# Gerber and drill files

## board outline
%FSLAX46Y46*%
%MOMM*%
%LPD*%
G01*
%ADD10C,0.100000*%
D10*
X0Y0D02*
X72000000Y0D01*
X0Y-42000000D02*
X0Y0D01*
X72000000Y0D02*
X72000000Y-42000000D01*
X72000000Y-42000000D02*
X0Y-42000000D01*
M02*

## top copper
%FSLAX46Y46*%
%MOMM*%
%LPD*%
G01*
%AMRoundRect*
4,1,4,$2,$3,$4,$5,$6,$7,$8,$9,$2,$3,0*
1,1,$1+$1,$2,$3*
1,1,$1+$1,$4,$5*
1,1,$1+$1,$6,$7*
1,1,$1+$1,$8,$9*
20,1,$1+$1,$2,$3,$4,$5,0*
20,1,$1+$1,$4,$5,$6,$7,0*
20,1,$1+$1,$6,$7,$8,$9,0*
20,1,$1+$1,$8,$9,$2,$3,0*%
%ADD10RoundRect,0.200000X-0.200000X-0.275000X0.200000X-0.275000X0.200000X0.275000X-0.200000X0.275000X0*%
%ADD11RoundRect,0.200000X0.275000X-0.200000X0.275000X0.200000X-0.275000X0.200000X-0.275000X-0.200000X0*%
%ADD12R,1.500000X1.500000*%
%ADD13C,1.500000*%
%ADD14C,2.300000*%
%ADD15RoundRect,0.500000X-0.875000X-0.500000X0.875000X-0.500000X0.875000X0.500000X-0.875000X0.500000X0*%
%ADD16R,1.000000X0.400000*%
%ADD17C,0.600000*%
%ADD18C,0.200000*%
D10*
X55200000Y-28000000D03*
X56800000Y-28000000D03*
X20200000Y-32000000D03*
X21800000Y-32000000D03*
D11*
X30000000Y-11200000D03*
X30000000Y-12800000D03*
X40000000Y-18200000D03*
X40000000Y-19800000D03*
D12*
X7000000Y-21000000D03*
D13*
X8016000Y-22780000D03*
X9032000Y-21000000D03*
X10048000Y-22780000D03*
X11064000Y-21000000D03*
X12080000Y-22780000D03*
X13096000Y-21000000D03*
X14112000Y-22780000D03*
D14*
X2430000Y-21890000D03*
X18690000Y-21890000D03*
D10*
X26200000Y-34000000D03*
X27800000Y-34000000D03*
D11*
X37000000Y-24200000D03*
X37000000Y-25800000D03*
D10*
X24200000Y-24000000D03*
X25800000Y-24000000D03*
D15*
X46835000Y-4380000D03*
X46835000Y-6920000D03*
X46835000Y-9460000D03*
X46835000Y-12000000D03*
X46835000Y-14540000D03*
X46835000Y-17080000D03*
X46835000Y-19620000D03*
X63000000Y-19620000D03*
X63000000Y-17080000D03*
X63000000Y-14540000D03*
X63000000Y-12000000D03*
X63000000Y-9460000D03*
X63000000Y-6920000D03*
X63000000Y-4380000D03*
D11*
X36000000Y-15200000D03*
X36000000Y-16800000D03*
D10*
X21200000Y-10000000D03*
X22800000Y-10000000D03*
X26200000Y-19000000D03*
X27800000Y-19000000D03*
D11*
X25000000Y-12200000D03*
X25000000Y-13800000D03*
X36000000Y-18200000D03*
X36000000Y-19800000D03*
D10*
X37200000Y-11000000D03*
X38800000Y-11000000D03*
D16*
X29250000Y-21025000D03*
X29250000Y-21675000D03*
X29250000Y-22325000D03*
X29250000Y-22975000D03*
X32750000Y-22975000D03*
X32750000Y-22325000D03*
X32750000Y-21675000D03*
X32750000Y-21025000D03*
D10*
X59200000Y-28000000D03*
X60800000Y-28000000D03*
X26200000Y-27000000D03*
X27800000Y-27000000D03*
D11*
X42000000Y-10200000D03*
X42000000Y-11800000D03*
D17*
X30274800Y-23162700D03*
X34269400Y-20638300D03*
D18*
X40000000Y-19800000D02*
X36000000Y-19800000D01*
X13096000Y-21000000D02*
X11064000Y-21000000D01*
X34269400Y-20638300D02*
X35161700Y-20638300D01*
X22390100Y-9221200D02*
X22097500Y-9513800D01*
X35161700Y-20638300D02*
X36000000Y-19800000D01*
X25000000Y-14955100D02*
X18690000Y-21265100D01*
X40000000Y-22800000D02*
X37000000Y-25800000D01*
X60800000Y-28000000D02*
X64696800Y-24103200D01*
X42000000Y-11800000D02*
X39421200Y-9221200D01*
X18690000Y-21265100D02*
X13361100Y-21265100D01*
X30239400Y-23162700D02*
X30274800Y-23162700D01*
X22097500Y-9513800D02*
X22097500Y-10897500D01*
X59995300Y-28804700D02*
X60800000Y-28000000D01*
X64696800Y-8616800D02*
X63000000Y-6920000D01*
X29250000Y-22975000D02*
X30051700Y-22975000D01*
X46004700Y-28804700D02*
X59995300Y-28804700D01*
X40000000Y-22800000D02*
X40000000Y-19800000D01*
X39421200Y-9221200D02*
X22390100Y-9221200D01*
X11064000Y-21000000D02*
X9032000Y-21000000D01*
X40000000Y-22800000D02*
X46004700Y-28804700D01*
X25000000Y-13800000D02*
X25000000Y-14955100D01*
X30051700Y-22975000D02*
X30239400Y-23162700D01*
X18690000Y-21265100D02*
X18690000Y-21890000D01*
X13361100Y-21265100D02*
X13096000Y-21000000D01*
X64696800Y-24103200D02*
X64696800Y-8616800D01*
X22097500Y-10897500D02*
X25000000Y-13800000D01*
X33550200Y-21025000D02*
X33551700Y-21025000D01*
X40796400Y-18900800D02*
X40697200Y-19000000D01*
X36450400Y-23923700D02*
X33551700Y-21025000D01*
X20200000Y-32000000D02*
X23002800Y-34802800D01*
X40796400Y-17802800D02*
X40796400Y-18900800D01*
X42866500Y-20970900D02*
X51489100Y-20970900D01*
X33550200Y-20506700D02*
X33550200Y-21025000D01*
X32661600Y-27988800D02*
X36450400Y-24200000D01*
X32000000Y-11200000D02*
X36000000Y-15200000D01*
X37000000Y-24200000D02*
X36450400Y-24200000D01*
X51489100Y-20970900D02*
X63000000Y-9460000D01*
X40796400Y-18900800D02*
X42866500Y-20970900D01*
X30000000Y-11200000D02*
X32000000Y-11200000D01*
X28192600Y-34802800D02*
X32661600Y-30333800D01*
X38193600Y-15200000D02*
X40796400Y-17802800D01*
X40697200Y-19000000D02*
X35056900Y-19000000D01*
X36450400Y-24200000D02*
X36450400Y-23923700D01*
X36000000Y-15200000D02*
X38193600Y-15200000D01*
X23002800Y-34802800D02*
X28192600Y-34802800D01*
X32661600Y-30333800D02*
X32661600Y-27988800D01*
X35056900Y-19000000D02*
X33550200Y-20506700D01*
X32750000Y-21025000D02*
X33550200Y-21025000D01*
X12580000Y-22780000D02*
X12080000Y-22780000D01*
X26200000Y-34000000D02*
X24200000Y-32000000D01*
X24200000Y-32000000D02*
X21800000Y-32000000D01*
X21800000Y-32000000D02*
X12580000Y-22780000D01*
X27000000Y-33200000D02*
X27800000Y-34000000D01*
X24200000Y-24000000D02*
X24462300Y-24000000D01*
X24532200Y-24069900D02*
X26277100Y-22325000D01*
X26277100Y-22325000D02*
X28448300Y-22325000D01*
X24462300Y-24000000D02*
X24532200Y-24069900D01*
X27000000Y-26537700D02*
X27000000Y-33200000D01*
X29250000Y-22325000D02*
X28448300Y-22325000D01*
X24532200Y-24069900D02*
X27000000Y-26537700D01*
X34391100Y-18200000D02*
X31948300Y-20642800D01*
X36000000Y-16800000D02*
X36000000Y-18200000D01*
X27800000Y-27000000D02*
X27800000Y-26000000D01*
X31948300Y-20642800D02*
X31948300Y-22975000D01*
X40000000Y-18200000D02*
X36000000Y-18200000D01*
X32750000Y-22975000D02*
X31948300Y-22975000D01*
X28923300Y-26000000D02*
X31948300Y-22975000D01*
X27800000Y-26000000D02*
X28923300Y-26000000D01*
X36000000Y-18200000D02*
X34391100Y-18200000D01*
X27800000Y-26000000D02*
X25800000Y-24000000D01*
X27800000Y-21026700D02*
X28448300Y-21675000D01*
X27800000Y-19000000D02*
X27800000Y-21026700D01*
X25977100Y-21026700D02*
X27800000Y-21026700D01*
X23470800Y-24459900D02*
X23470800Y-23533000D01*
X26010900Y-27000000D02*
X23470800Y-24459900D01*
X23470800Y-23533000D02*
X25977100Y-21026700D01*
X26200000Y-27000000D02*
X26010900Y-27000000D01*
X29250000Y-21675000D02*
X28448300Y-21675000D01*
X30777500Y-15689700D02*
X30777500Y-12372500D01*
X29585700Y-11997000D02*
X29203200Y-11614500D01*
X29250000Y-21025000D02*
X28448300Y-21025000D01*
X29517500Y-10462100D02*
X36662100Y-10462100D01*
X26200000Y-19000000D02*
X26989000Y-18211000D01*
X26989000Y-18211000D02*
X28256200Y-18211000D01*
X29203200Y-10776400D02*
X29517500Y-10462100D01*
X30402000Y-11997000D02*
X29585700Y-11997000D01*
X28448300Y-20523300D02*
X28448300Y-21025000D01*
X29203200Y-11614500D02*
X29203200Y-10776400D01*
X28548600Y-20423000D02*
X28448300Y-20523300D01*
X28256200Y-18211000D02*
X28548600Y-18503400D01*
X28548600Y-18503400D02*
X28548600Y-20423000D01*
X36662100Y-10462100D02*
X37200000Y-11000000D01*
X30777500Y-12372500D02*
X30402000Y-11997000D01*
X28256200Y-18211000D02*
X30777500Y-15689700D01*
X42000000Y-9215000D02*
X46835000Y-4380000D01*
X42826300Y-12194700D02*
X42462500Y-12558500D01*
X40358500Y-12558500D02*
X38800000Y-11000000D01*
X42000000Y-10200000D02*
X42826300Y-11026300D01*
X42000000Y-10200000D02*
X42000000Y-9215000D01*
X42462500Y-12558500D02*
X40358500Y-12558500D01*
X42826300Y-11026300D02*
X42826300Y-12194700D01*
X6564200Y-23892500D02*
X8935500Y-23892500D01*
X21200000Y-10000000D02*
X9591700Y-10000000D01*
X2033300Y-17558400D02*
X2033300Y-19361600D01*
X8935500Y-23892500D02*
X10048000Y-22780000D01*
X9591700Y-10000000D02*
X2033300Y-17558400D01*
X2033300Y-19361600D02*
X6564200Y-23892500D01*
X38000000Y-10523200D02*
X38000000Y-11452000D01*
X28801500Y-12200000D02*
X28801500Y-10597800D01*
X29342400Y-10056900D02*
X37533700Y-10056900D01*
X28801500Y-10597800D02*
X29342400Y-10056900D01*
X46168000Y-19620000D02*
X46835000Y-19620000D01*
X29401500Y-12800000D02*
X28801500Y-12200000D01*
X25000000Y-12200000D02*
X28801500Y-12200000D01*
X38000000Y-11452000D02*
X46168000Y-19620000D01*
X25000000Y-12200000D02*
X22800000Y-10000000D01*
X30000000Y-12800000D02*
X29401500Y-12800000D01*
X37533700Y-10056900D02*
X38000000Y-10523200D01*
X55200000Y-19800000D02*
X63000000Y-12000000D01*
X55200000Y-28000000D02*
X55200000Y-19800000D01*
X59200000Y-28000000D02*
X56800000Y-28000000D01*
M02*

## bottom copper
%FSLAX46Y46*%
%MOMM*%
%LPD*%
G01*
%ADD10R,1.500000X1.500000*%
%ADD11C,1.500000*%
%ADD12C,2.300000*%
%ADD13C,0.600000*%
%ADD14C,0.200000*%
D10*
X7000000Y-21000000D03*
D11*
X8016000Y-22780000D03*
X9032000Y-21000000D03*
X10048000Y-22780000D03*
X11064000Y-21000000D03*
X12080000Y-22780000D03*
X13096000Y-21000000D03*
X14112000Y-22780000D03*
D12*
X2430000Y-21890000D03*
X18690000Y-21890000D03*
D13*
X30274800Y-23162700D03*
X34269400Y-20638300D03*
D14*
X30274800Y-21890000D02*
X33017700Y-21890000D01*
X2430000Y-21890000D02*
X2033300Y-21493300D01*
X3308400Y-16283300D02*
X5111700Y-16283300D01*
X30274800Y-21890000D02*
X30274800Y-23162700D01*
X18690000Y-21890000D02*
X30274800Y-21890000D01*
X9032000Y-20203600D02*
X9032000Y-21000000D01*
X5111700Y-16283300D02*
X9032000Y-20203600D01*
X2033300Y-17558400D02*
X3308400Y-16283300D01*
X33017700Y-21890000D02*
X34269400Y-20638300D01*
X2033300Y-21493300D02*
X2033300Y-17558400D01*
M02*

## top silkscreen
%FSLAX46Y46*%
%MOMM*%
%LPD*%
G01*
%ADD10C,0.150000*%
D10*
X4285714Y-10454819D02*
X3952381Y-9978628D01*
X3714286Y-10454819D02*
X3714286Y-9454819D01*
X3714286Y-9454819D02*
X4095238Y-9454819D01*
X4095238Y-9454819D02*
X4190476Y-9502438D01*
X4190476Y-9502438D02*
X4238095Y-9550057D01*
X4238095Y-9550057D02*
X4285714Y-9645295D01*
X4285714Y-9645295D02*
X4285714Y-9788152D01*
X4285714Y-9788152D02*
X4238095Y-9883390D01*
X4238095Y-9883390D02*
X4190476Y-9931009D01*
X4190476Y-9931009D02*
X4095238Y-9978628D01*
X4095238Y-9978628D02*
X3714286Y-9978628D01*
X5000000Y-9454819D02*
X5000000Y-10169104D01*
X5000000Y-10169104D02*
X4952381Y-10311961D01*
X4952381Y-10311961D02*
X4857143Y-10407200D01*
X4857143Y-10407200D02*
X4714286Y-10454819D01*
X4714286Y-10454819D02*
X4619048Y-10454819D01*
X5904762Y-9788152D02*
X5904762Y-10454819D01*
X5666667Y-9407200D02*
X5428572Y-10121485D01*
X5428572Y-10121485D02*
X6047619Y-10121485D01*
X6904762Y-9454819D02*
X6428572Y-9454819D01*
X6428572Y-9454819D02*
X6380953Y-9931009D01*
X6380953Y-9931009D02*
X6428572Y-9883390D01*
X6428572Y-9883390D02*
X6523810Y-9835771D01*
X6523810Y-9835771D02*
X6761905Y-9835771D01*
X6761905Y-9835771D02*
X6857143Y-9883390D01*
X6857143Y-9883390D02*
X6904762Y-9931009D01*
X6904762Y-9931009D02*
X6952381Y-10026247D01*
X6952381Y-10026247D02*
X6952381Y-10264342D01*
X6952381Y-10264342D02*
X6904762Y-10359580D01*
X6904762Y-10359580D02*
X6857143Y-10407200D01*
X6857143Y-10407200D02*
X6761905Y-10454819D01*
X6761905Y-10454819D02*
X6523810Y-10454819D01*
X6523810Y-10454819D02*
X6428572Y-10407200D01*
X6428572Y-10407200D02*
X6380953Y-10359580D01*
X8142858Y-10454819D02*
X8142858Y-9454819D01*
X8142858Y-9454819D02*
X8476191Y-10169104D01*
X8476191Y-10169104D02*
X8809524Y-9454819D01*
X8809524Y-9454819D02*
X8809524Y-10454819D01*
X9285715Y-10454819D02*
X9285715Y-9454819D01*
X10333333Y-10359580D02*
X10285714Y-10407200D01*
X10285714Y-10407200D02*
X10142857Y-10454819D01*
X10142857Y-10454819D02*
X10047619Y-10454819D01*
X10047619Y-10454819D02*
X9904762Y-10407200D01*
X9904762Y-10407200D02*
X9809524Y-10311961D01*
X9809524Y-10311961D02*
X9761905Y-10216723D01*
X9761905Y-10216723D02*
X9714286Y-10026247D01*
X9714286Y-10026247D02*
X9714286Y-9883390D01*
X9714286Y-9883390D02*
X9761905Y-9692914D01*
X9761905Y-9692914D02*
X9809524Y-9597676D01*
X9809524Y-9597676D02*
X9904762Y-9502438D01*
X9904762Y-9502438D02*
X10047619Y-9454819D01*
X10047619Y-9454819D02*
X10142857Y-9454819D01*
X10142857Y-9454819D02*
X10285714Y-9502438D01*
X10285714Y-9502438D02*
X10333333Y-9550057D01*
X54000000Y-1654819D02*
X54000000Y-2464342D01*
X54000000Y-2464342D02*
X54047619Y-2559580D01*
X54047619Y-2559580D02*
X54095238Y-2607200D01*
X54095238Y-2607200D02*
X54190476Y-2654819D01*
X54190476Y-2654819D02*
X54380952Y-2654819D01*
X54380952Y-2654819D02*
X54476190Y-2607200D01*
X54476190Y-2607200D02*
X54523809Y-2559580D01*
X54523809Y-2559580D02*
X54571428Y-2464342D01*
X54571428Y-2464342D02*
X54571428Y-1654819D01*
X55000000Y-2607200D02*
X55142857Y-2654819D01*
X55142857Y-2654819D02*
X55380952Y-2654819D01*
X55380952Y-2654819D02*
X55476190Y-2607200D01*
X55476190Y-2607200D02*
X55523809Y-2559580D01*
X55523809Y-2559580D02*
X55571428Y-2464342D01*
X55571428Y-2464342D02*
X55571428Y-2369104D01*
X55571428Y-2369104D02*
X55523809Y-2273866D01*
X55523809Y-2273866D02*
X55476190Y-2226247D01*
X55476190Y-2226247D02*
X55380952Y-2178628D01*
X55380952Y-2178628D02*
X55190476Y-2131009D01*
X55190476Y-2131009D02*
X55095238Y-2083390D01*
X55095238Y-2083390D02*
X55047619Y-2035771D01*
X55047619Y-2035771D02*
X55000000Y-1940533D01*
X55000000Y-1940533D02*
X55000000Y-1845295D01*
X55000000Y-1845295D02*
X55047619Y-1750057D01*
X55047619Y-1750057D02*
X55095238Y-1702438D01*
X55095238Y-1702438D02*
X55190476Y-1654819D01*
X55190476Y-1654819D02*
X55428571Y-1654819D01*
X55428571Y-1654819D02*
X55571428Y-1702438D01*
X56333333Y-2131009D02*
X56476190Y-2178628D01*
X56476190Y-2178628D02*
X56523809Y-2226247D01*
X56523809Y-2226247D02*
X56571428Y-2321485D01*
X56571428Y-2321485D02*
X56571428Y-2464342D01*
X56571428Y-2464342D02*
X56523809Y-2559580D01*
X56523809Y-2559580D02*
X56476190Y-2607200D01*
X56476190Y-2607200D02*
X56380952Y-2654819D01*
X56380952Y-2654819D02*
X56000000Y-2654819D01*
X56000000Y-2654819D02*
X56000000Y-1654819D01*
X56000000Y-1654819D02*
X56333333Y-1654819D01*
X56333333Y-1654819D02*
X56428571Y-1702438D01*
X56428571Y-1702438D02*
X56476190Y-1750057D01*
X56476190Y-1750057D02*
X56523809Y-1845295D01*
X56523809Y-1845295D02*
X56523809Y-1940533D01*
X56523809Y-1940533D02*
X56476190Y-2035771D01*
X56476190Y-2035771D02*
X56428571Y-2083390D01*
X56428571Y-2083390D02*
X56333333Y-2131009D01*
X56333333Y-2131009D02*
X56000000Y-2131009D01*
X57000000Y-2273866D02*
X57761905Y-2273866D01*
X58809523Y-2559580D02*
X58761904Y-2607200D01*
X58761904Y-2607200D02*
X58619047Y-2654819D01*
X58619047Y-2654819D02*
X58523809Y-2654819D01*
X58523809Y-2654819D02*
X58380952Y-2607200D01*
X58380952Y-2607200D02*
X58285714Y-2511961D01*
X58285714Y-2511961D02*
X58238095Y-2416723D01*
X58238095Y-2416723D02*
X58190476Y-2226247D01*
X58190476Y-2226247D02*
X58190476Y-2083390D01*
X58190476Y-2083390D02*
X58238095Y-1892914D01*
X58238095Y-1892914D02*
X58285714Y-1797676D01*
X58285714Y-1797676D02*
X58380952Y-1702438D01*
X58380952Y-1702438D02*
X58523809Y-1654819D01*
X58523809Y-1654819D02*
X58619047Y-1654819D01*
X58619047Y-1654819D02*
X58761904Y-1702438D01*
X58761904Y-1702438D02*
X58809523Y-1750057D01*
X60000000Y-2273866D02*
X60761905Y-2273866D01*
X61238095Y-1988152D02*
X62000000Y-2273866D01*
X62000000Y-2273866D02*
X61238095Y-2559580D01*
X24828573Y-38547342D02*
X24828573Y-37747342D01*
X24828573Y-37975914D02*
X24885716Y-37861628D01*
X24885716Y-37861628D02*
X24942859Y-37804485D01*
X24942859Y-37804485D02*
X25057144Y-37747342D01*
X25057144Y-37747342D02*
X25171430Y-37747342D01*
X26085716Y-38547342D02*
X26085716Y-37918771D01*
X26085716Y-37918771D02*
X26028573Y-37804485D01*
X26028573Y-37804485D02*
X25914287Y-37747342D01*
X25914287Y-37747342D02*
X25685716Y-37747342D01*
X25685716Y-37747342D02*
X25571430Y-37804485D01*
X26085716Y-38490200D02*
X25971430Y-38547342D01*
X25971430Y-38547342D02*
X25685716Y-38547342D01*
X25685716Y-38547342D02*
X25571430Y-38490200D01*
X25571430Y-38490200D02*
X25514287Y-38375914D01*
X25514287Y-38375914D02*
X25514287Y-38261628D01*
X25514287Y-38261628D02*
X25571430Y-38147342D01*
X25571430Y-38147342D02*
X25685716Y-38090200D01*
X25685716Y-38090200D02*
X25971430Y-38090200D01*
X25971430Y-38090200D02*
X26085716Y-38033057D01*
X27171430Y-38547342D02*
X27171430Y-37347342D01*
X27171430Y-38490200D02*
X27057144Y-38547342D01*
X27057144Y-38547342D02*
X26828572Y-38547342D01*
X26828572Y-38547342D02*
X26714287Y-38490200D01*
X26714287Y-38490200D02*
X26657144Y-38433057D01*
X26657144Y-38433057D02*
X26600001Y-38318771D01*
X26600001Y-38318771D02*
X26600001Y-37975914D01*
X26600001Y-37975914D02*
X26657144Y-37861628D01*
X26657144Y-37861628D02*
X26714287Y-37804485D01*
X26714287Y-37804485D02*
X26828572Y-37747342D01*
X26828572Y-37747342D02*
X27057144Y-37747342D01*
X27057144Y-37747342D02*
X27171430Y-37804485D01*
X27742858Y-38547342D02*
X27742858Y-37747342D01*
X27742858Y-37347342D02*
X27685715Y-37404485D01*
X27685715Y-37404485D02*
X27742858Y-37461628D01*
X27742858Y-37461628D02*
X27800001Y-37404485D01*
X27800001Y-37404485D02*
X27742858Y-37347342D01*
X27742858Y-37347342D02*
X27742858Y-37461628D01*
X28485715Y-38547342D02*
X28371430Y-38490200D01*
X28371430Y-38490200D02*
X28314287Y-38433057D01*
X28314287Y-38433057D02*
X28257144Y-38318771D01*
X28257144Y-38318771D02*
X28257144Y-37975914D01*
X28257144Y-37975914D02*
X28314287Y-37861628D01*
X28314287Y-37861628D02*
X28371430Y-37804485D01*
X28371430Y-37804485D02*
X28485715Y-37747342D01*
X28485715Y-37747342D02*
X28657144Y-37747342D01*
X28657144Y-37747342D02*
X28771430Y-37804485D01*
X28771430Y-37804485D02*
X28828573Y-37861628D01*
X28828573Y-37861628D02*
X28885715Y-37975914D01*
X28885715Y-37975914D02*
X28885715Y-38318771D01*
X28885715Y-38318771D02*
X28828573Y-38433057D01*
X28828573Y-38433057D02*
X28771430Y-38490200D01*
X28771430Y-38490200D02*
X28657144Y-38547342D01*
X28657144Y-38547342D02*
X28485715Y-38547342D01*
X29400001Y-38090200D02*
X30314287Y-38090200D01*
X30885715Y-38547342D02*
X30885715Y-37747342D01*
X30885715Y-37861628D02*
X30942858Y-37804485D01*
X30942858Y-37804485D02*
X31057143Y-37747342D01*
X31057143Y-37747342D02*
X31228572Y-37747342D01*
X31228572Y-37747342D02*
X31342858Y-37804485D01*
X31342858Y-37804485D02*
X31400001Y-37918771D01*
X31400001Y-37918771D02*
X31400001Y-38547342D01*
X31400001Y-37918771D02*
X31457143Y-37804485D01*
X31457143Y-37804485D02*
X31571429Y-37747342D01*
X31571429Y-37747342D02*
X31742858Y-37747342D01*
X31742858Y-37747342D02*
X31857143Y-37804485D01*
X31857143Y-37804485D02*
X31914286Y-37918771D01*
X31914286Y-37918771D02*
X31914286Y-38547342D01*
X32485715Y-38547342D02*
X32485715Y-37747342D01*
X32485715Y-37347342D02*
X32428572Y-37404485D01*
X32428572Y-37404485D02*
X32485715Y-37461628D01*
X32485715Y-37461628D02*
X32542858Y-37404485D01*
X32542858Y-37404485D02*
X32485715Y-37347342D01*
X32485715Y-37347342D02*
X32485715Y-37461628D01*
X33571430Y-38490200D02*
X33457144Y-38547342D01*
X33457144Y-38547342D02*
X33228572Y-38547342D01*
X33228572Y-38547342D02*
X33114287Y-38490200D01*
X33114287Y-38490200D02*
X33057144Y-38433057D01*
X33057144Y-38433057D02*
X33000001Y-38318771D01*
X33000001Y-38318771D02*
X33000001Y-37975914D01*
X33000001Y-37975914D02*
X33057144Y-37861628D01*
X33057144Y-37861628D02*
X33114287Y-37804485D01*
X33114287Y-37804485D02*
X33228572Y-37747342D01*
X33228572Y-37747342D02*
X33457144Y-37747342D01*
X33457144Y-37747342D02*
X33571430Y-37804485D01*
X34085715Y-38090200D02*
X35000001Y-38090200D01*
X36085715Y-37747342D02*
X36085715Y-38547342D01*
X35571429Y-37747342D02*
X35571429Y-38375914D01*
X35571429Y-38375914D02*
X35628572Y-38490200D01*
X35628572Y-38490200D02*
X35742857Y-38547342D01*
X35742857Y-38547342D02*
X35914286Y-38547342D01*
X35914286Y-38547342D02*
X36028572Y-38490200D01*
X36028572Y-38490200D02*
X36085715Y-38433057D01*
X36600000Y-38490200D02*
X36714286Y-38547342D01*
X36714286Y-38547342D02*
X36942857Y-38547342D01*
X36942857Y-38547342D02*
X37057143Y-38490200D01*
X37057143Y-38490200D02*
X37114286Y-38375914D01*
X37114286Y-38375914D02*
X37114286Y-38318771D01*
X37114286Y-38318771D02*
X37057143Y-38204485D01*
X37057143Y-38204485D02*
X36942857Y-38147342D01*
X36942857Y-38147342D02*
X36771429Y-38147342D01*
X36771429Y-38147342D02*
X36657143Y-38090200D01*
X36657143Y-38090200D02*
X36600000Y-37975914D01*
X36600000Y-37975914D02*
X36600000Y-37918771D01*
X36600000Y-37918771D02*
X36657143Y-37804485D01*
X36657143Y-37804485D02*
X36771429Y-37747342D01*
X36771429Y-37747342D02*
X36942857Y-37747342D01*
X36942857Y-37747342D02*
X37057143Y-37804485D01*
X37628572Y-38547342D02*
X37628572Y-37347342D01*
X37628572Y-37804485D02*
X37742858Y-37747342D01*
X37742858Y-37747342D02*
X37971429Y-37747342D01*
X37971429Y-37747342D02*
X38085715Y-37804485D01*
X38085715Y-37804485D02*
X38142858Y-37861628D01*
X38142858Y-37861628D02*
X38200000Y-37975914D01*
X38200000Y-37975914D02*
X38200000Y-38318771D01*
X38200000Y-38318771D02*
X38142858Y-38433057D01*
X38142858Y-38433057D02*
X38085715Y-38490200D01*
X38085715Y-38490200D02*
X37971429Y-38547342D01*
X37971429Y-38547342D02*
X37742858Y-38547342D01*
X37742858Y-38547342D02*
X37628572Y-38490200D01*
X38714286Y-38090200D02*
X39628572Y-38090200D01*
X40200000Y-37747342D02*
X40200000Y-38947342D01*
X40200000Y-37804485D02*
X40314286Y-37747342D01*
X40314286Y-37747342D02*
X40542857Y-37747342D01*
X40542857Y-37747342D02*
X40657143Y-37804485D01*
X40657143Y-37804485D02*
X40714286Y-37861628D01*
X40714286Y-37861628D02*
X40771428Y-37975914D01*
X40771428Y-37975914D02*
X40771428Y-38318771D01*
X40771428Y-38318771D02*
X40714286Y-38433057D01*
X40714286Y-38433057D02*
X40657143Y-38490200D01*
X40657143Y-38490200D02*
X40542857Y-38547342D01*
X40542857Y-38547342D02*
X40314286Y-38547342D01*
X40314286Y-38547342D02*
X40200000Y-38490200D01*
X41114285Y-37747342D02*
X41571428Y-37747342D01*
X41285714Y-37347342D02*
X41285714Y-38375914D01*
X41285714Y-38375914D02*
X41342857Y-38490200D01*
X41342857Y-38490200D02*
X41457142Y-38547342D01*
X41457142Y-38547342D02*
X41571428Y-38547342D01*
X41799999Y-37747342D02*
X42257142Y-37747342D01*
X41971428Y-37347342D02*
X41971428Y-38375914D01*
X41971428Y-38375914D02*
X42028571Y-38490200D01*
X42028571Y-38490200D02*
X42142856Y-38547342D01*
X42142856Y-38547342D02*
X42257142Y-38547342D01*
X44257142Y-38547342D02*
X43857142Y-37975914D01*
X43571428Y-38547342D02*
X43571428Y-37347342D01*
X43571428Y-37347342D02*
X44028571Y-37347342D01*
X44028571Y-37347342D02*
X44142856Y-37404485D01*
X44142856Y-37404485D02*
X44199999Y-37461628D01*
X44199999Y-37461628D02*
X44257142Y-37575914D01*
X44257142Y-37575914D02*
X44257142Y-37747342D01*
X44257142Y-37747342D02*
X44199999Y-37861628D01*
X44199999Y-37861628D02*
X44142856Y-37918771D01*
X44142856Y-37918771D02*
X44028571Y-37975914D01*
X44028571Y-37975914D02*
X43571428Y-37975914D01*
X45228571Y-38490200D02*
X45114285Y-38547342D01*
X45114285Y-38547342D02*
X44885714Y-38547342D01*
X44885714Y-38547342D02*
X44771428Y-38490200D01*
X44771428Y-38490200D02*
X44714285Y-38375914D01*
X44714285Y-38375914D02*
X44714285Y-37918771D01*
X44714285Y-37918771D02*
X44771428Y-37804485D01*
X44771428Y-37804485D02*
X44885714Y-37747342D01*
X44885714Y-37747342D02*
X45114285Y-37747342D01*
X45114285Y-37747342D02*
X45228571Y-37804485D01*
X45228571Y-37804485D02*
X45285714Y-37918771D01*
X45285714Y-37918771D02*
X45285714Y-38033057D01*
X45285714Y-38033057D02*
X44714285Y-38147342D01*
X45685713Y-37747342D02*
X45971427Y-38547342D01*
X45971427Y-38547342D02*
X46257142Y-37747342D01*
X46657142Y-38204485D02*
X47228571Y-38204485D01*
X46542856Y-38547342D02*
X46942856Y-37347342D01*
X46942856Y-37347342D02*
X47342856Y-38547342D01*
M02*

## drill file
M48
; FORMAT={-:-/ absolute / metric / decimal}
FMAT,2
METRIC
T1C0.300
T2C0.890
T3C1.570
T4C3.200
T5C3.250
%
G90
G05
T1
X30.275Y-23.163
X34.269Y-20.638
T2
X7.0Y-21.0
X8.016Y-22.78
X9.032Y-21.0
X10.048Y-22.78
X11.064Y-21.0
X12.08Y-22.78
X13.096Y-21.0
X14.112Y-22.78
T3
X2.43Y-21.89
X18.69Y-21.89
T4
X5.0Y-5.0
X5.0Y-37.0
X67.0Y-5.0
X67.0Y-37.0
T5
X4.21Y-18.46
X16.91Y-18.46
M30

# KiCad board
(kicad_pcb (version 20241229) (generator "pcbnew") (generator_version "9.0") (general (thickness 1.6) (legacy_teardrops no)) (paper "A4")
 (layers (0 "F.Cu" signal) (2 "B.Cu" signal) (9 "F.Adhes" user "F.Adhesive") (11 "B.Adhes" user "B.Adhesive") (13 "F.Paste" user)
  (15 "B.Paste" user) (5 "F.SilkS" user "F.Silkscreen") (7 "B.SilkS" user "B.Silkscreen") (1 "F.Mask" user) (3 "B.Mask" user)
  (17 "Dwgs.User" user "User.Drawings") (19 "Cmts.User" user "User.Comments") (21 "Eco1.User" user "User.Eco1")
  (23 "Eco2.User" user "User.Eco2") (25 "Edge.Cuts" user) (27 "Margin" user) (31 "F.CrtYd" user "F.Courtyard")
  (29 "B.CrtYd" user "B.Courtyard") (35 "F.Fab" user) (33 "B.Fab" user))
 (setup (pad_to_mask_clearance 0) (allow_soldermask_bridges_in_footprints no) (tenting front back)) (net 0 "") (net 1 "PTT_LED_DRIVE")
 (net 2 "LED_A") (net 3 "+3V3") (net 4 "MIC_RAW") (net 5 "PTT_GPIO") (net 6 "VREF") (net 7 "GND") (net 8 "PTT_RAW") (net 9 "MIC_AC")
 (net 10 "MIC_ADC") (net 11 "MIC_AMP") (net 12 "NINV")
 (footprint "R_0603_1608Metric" (layer "F.Cu") (at 56 28)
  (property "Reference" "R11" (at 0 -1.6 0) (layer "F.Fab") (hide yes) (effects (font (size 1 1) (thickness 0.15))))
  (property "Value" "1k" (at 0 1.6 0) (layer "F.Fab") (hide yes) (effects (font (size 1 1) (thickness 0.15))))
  (pad "1" smd roundrect (at -0.8 0) (size 0.8 0.95) (layers "F.Cu" "F.Mask" "F.Paste") (roundrect_rratio 0.25) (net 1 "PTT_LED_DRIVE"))
  (pad "2" smd roundrect (at 0.8 0) (size 0.8 0.95) (layers "F.Cu" "F.Mask" "F.Paste") (roundrect_rratio 0.25) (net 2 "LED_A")))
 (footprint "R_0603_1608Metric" (layer "F.Cu") (at 21 32)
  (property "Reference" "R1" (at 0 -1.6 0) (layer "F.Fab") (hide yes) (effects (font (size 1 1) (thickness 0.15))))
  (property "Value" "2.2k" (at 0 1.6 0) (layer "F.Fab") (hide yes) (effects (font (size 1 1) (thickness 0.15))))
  (pad "1" smd roundrect (at -0.8 0) (size 0.8 0.95) (layers "F.Cu" "F.Mask" "F.Paste") (roundrect_rratio 0.25) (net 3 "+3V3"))
  (pad "2" smd roundrect (at 0.8 0) (size 0.8 0.95) (layers "F.Cu" "F.Mask" "F.Paste") (roundrect_rratio 0.25) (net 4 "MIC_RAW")))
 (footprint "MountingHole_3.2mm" (layer "F.Cu") (at 67 37)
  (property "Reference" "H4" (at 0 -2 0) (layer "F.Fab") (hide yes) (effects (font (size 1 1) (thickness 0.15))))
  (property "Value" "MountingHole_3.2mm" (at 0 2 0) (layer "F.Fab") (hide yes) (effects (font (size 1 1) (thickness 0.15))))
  (pad "" np_thru_hole circle (at 0 0) (size 3.2 3.2) (drill 3.2) (layers "*.Cu" "*.Mask")))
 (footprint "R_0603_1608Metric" (layer "F.Cu") (at 30 12)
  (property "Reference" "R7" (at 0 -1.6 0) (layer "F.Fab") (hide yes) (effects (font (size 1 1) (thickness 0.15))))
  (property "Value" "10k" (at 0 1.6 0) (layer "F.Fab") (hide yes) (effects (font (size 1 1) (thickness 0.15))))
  (pad "1" smd roundrect (at 0 -0.8 90) (size 0.8 0.95) (layers "F.Cu" "F.Mask" "F.Paste") (roundrect_rratio 0.25) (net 3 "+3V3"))
  (pad "2" smd roundrect (at 0 0.8 90) (size 0.8 0.95) (layers "F.Cu" "F.Mask" "F.Paste") (roundrect_rratio 0.25) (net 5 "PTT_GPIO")))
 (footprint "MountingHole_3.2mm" (layer "F.Cu") (at 67 5)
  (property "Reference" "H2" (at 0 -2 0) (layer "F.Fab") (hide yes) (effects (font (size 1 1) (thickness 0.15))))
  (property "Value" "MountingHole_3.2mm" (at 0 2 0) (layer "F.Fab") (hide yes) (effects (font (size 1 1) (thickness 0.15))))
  (pad "" np_thru_hole circle (at 0 0) (size 3.2 3.2) (drill 3.2) (layers "*.Cu" "*.Mask")))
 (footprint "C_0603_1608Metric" (layer "F.Cu") (at 40 19)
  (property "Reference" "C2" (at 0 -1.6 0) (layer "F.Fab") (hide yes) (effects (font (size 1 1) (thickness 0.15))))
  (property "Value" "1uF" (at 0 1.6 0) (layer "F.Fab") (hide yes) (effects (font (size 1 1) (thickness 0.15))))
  (pad "1" smd roundrect (at 0 -0.8 90) (size 0.8 0.95) (layers "F.Cu" "F.Mask" "F.Paste") (roundrect_rratio 0.25) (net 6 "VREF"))
  (pad "2" smd roundrect (at 0 0.8 90) (size 0.8 0.95) (layers "F.Cu" "F.Mask" "F.Paste") (roundrect_rratio 0.25) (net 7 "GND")))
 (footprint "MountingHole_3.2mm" (layer "F.Cu") (at 5 37)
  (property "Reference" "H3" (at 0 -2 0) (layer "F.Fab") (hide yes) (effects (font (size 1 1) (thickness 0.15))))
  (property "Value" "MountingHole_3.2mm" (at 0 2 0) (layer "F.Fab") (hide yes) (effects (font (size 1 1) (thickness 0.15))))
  (pad "" np_thru_hole circle (at 0 0) (size 3.2 3.2) (drill 3.2) (layers "*.Cu" "*.Mask")))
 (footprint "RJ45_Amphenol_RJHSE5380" (layer "F.Cu") (at 7 21)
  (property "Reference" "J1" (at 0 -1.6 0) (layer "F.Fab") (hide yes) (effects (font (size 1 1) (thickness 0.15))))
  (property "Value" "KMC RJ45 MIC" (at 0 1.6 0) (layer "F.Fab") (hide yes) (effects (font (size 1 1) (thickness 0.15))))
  (pad "" np_thru_hole circle (at -2.79 -2.54) (size 3.25 3.25) (drill 3.25) (layers "*.Cu" "*.Mask"))
  (pad "" np_thru_hole circle (at 9.91 -2.54) (size 3.25 3.25) (drill 3.25) (layers "*.Cu" "*.Mask"))
  (pad "1" thru_hole rect (at 0 0) (size 1.5 1.5) (drill 0.89) (layers "*.Cu" "*.Mask") (remove_unused_layers no))
  (pad "2" thru_hole circle (at 1.016 1.78) (size 1.5 1.5) (drill 0.89) (layers "*.Cu" "*.Mask") (remove_unused_layers no))
  (pad "3" thru_hole circle (at 2.032 0) (size 1.5 1.5) (drill 0.89) (layers "*.Cu" "*.Mask") (remove_unused_layers no) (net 7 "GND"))
  (pad "4" thru_hole circle (at 3.048 1.78) (size 1.5 1.5) (drill 0.89) (layers "*.Cu" "*.Mask") (remove_unused_layers no) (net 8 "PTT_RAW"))
  (pad "5" thru_hole circle (at 4.064 0) (size 1.5 1.5) (drill 0.89) (layers "*.Cu" "*.Mask") (remove_unused_layers no) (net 7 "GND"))
  (pad "6" thru_hole circle (at 5.08 1.78) (size 1.5 1.5) (drill 0.89) (layers "*.Cu" "*.Mask") (remove_unused_layers no) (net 4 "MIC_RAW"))
  (pad "7" thru_hole circle (at 6.096 0) (size 1.5 1.5) (drill 0.89) (layers "*.Cu" "*.Mask") (remove_unused_layers no) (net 7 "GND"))
  (pad "8" thru_hole circle (at 7.112 1.78) (size 1.5 1.5) (drill 0.89) (layers "*.Cu" "*.Mask") (remove_unused_layers no))
  (pad "SH" thru_hole circle (at -4.57 0.89) (size 2.3 2.3) (drill 1.57) (layers "*.Cu" "*.Mask") (remove_unused_layers no) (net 7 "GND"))
  (pad "SH" thru_hole circle (at 11.69 0.89) (size 2.3 2.3) (drill 1.57) (layers "*.Cu" "*.Mask") (remove_unused_layers no) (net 7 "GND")))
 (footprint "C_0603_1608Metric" (layer "F.Cu") (at 27 34)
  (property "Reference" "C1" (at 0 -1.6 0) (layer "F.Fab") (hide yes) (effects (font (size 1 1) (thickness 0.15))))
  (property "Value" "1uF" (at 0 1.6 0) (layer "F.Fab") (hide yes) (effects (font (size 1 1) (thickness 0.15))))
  (pad "1" smd roundrect (at -0.8 0) (size 0.8 0.95) (layers "F.Cu" "F.Mask" "F.Paste") (roundrect_rratio 0.25) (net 4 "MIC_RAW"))
  (pad "2" smd roundrect (at 0.8 0) (size 0.8 0.95) (layers "F.Cu" "F.Mask" "F.Paste") (roundrect_rratio 0.25) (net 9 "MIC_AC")))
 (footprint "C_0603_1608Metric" (layer "F.Cu") (at 37 25)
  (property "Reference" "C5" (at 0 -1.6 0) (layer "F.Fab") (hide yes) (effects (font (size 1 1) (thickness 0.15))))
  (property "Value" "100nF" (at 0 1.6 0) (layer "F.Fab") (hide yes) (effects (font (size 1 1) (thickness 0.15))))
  (pad "1" smd roundrect (at 0 -0.8 90) (size 0.8 0.95) (layers "F.Cu" "F.Mask" "F.Paste") (roundrect_rratio 0.25) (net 3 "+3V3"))
  (pad "2" smd roundrect (at 0 0.8 90) (size 0.8 0.95) (layers "F.Cu" "F.Mask" "F.Paste") (roundrect_rratio 0.25) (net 7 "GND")))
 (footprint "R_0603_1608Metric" (layer "F.Cu") (at 25 24)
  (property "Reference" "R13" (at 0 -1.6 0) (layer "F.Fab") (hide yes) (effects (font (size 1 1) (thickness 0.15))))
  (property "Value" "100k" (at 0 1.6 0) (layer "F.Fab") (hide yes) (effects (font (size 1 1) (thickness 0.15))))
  (pad "1" smd roundrect (at -0.8 0) (size 0.8 0.95) (layers "F.Cu" "F.Mask" "F.Paste") (roundrect_rratio 0.25) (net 9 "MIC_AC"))
  (pad "2" smd roundrect (at 0.8 0) (size 0.8 0.95) (layers "F.Cu" "F.Mask" "F.Paste") (roundrect_rratio 0.25) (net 6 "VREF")))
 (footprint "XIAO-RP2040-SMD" (layer "F.Cu") (at 46 22.5)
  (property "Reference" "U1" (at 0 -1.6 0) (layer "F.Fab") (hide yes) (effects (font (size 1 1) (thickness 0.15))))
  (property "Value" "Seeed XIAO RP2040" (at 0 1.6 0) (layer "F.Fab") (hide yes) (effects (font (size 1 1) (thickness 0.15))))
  (pad "1" smd roundrect (at 0.835 -18.12) (size 2.75 2) (layers "F.Cu" "F.Mask" "F.Paste") (roundrect_rratio 0.25) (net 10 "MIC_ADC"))
  (pad "2" smd roundrect (at 0.835 -15.58) (size 2.75 2) (layers "F.Cu" "F.Mask" "F.Paste") (roundrect_rratio 0.25))
  (pad "3" smd roundrect (at 0.835 -13.04) (size 2.75 2) (layers "F.Cu" "F.Mask" "F.Paste") (roundrect_rratio 0.25))
  (pad "4" smd roundrect (at 0.835 -10.5) (size 2.75 2) (layers "F.Cu" "F.Mask" "F.Paste") (roundrect_rratio 0.25))
  (pad "5" smd roundrect (at 0.835 -7.96) (size 2.75 2) (layers "F.Cu" "F.Mask" "F.Paste") (roundrect_rratio 0.25))
  (pad "6" smd roundrect (at 0.835 -5.42) (size 2.75 2) (layers "F.Cu" "F.Mask" "F.Paste") (roundrect_rratio 0.25))
  (pad "7" smd roundrect (at 0.835 -2.88) (size 2.75 2) (layers "F.Cu" "F.Mask" "F.Paste") (roundrect_rratio 0.25) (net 5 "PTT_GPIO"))
  (pad "8" smd roundrect (at 17 -2.88) (size 2.75 2) (layers "F.Cu" "F.Mask" "F.Paste") (roundrect_rratio 0.25))
  (pad "9" smd roundrect (at 17 -5.42) (size 2.75 2) (layers "F.Cu" "F.Mask" "F.Paste") (roundrect_rratio 0.25))
  (pad "10" smd roundrect (at 17 -7.96) (size 2.75 2) (layers "F.Cu" "F.Mask" "F.Paste") (roundrect_rratio 0.25))
  (pad "11" smd roundrect (at 17 -10.5) (size 2.75 2) (layers "F.Cu" "F.Mask" "F.Paste") (roundrect_rratio 0.25) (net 1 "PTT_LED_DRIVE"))
  (pad "12" smd roundrect (at 17 -13.04) (size 2.75 2) (layers "F.Cu" "F.Mask" "F.Paste") (roundrect_rratio 0.25) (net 3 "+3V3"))
  (pad "13" smd roundrect (at 17 -15.58) (size 2.75 2) (layers "F.Cu" "F.Mask" "F.Paste") (roundrect_rratio 0.25) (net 7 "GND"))
  (pad "14" smd roundrect (at 17 -18.12) (size 2.75 2) (layers "F.Cu" "F.Mask" "F.Paste") (roundrect_rratio 0.25)))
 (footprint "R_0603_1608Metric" (layer "F.Cu") (at 36 16)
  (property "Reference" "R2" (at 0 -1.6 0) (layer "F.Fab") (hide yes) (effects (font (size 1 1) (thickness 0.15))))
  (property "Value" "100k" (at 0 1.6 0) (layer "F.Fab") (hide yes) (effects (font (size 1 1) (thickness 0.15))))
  (pad "1" smd roundrect (at 0 -0.8 90) (size 0.8 0.95) (layers "F.Cu" "F.Mask" "F.Paste") (roundrect_rratio 0.25) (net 3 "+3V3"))
  (pad "2" smd roundrect (at 0 0.8 90) (size 0.8 0.95) (layers "F.Cu" "F.Mask" "F.Paste") (roundrect_rratio 0.25) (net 6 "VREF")))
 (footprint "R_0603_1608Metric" (layer "F.Cu") (at 22 10)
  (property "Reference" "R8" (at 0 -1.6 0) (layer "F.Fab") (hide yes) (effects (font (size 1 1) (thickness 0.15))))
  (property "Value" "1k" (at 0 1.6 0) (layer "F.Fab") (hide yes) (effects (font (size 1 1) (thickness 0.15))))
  (pad "1" smd roundrect (at -0.8 0) (size 0.8 0.95) (layers "F.Cu" "F.Mask" "F.Paste") (roundrect_rratio 0.25) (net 8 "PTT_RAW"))
  (pad "2" smd roundrect (at 0.8 0) (size 0.8 0.95) (layers "F.Cu" "F.Mask" "F.Paste") (roundrect_rratio 0.25) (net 5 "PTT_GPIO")))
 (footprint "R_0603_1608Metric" (layer "F.Cu") (at 27 19)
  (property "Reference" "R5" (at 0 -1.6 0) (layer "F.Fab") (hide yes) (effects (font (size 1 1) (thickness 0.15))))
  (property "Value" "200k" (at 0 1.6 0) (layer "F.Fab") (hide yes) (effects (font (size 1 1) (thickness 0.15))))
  (pad "1" smd roundrect (at -0.8 0) (size 0.8 0.95) (layers "F.Cu" "F.Mask" "F.Paste") (roundrect_rratio 0.25) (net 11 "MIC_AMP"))
  (pad "2" smd roundrect (at 0.8 0) (size 0.8 0.95) (layers "F.Cu" "F.Mask" "F.Paste") (roundrect_rratio 0.25) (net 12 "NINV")))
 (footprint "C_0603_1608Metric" (layer "F.Cu") (at 25 13)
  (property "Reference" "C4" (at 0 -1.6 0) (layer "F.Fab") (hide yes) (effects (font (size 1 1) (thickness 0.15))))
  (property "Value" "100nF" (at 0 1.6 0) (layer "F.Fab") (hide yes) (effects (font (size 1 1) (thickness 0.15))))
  (pad "1" smd roundrect (at 0 -0.8 90) (size 0.8 0.95) (layers "F.Cu" "F.Mask" "F.Paste") (roundrect_rratio 0.25) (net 5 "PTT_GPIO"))
  (pad "2" smd roundrect (at 0 0.8 90) (size 0.8 0.95) (layers "F.Cu" "F.Mask" "F.Paste") (roundrect_rratio 0.25) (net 7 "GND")))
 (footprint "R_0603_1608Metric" (layer "F.Cu") (at 36 19)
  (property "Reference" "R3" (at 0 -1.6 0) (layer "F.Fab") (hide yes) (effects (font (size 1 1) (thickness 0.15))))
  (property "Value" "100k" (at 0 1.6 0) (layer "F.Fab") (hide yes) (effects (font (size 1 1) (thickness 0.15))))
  (pad "1" smd roundrect (at 0 -0.8 90) (size 0.8 0.95) (layers "F.Cu" "F.Mask" "F.Paste") (roundrect_rratio 0.25) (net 6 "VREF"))
  (pad "2" smd roundrect (at 0 0.8 90) (size 0.8 0.95) (layers "F.Cu" "F.Mask" "F.Paste") (roundrect_rratio 0.25) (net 7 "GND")))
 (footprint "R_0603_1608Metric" (layer "F.Cu") (at 38 11)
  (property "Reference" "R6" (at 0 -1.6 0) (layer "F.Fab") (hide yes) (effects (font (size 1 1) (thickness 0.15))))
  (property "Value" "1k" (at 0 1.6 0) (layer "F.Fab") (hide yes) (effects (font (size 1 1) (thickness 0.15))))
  (pad "1" smd roundrect (at -0.8 0) (size 0.8 0.95) (layers "F.Cu" "F.Mask" "F.Paste") (roundrect_rratio 0.25) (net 11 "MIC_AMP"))
  (pad "2" smd roundrect (at 0.8 0) (size 0.8 0.95) (layers "F.Cu" "F.Mask" "F.Paste") (roundrect_rratio 0.25) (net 10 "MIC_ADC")))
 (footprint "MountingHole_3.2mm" (layer "F.Cu") (at 5 5)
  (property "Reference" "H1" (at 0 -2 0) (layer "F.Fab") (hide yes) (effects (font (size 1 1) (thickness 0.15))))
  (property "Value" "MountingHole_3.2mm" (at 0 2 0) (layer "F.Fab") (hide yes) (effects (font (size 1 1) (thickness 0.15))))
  (pad "" np_thru_hole circle (at 0 0) (size 3.2 3.2) (drill 3.2) (layers "*.Cu" "*.Mask")))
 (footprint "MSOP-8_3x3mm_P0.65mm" (layer "F.Cu") (at 31 22)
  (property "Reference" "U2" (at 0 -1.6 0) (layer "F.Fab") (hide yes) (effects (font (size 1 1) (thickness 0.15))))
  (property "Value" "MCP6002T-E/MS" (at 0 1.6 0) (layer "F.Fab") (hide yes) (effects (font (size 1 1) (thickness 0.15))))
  (pad "1" smd rect (at -1.75 -0.975) (size 1 0.4) (layers "F.Cu" "F.Mask" "F.Paste") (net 11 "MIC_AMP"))
  (pad "2" smd rect (at -1.75 -0.325) (size 1 0.4) (layers "F.Cu" "F.Mask" "F.Paste") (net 12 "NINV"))
  (pad "3" smd rect (at -1.75 0.325) (size 1 0.4) (layers "F.Cu" "F.Mask" "F.Paste") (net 9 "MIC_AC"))
  (pad "4" smd rect (at -1.75 0.975) (size 1 0.4) (layers "F.Cu" "F.Mask" "F.Paste") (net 7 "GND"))
  (pad "5" smd rect (at 1.75 0.975) (size 1 0.4) (layers "F.Cu" "F.Mask" "F.Paste") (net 6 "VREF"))
  (pad "6" smd rect (at 1.75 0.325) (size 1 0.4) (layers "F.Cu" "F.Mask" "F.Paste"))
  (pad "7" smd rect (at 1.75 -0.325) (size 1 0.4) (layers "F.Cu" "F.Mask" "F.Paste"))
  (pad "8" smd rect (at 1.75 -0.975) (size 1 0.4) (layers "F.Cu" "F.Mask" "F.Paste") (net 3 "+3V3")))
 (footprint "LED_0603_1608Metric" (layer "F.Cu") (at 60 28)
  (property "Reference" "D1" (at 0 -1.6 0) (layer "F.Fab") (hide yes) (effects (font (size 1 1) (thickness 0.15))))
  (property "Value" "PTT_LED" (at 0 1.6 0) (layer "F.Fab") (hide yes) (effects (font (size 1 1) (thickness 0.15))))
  (pad "1" smd roundrect (at -0.8 0) (size 0.8 0.95) (layers "F.Cu" "F.Mask" "F.Paste") (roundrect_rratio 0.25) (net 2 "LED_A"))
  (pad "2" smd roundrect (at 0.8 0) (size 0.8 0.95) (layers "F.Cu" "F.Mask" "F.Paste") (roundrect_rratio 0.25) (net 7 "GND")))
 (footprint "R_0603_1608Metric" (layer "F.Cu") (at 27 27)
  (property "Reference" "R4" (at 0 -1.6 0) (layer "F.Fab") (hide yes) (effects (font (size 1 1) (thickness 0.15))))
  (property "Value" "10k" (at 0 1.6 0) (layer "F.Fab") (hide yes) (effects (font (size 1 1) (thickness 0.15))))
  (pad "1" smd roundrect (at -0.8 0) (size 0.8 0.95) (layers "F.Cu" "F.Mask" "F.Paste") (roundrect_rratio 0.25) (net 12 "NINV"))
  (pad "2" smd roundrect (at 0.8 0) (size 0.8 0.95) (layers "F.Cu" "F.Mask" "F.Paste") (roundrect_rratio 0.25) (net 6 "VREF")))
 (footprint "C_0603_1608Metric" (layer "F.Cu") (at 42 11)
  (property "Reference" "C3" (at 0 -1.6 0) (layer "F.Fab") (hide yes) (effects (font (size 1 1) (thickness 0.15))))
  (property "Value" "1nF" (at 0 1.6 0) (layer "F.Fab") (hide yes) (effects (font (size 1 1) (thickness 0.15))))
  (pad "1" smd roundrect (at 0 -0.8 90) (size 0.8 0.95) (layers "F.Cu" "F.Mask" "F.Paste") (roundrect_rratio 0.25) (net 10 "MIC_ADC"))
  (pad "2" smd roundrect (at 0 0.8 90) (size 0.8 0.95) (layers "F.Cu" "F.Mask" "F.Paste") (roundrect_rratio 0.25) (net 7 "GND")))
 (gr_line (start 0 0) (end 72 0) (stroke (width 0.1) (type default)) (layer "Edge.Cuts"))
 (gr_line (start 0 42) (end 0 0) (stroke (width 0.1) (type default)) (layer "Edge.Cuts"))
 (gr_line (start 72 0) (end 72 42) (stroke (width 0.1) (type default)) (layer "Edge.Cuts"))
 (gr_line (start 72 42) (end 0 42) (stroke (width 0.1) (type default)) (layer "Edge.Cuts"))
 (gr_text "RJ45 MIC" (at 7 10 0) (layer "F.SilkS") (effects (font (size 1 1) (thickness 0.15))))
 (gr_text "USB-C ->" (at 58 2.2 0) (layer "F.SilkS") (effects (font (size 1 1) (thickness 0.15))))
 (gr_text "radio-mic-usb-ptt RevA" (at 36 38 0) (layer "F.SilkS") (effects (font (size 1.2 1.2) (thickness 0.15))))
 (segment (start 40 19.8) (end 36 19.8) (width 0.2) (layer "F.Cu") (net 7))
 (segment (start 13.096 21) (end 11.064 21) (width 0.2) (layer "F.Cu") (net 7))
 (segment (start 34.2694 20.6383) (end 35.1617 20.6383) (width 0.2) (layer "F.Cu") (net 7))
 (segment (start 22.3901 9.2212) (end 22.0975 9.5138) (width 0.2) (layer "F.Cu") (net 7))
 (segment (start 35.1617 20.6383) (end 36 19.8) (width 0.2) (layer "F.Cu") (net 7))
 (segment (start 25 14.9551) (end 18.69 21.2651) (width 0.2) (layer "F.Cu") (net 7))
 (segment (start 40 22.8) (end 37 25.8) (width 0.2) (layer "F.Cu") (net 7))
 (segment (start 60.8 28) (end 64.6968 24.1032) (width 0.2) (layer "F.Cu") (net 7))
 (segment (start 42 11.8) (end 39.4212 9.2212) (width 0.2) (layer "F.Cu") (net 7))
 (segment (start 18.69 21.2651) (end 13.3611 21.2651) (width 0.2) (layer "F.Cu") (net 7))
 (segment (start 30.2394 23.1627) (end 30.2748 23.1627) (width 0.2) (layer "F.Cu") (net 7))
 (segment (start 22.0975 9.5138) (end 22.0975 10.8975) (width 0.2) (layer "F.Cu") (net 7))
 (segment (start 59.9953 28.8047) (end 60.8 28) (width 0.2) (layer "F.Cu") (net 7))
 (segment (start 64.6968 8.6168) (end 63 6.92) (width 0.2) (layer "F.Cu") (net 7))
 (segment (start 29.25 22.975) (end 30.0517 22.975) (width 0.2) (layer "F.Cu") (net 7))
 (segment (start 46.0047 28.8047) (end 59.9953 28.8047) (width 0.2) (layer "F.Cu") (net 7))
 (segment (start 40 22.8) (end 40 19.8) (width 0.2) (layer "F.Cu") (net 7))
 (segment (start 39.4212 9.2212) (end 22.3901 9.2212) (width 0.2) (layer "F.Cu") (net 7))
 (segment (start 11.064 21) (end 9.032 21) (width 0.2) (layer "F.Cu") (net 7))
 (segment (start 40 22.8) (end 46.0047 28.8047) (width 0.2) (layer "F.Cu") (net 7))
 (segment (start 25 13.8) (end 25 14.9551) (width 0.2) (layer "F.Cu") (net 7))
 (segment (start 30.0517 22.975) (end 30.2394 23.1627) (width 0.2) (layer "F.Cu") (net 7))
 (segment (start 18.69 21.2651) (end 18.69 21.89) (width 0.2) (layer "F.Cu") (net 7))
 (segment (start 13.3611 21.2651) (end 13.096 21) (width 0.2) (layer "F.Cu") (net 7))
 (segment (start 64.6968 24.1032) (end 64.6968 8.6168) (width 0.2) (layer "F.Cu") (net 7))
 (segment (start 22.0975 10.8975) (end 25 13.8) (width 0.2) (layer "F.Cu") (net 7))
 (via (at 30.2748 23.1627) (size 0.6) (drill 0.3) (layers "F.Cu" "B.Cu") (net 7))
 (via (at 34.2694 20.6383) (size 0.6) (drill 0.3) (layers "F.Cu" "B.Cu") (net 7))
 (segment (start 30.2748 21.89) (end 33.0177 21.89) (width 0.2) (layer "B.Cu") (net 7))
 (segment (start 2.43 21.89) (end 2.0333 21.4933) (width 0.2) (layer "B.Cu") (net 7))
 (segment (start 3.3084 16.2833) (end 5.1117 16.2833) (width 0.2) (layer "B.Cu") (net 7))
 (segment (start 30.2748 21.89) (end 30.2748 23.1627) (width 0.2) (layer "B.Cu") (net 7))
 (segment (start 18.69 21.89) (end 30.2748 21.89) (width 0.2) (layer "B.Cu") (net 7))
 (segment (start 9.032 20.2036) (end 9.032 21) (width 0.2) (layer "B.Cu") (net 7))
 (segment (start 5.1117 16.2833) (end 9.032 20.2036) (width 0.2) (layer "B.Cu") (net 7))
 (segment (start 2.0333 17.5584) (end 3.3084 16.2833) (width 0.2) (layer "B.Cu") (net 7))
 (segment (start 33.0177 21.89) (end 34.2694 20.6383) (width 0.2) (layer "B.Cu") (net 7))
 (segment (start 2.0333 21.4933) (end 2.0333 17.5584) (width 0.2) (layer "B.Cu") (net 7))
 (segment (start 33.5502 21.025) (end 33.5517 21.025) (width 0.2) (layer "F.Cu") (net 3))
 (segment (start 40.7964 18.9008) (end 40.6972 19) (width 0.2) (layer "F.Cu") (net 3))
 (segment (start 36.4504 23.9237) (end 33.5517 21.025) (width 0.2) (layer "F.Cu") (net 3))
 (segment (start 20.2 32) (end 23.0028 34.8028) (width 0.2) (layer "F.Cu") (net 3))
 (segment (start 40.7964 17.8028) (end 40.7964 18.9008) (width 0.2) (layer "F.Cu") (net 3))
 (segment (start 42.8665 20.9709) (end 51.4891 20.9709) (width 0.2) (layer "F.Cu") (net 3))
 (segment (start 33.5502 20.5067) (end 33.5502 21.025) (width 0.2) (layer "F.Cu") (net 3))
 (segment (start 32.6616 27.9888) (end 36.4504 24.2) (width 0.2) (layer "F.Cu") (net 3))
 (segment (start 32 11.2) (end 36 15.2) (width 0.2) (layer "F.Cu") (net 3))
 (segment (start 37 24.2) (end 36.4504 24.2) (width 0.2) (layer "F.Cu") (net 3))
 (segment (start 51.4891 20.9709) (end 63 9.46) (width 0.2) (layer "F.Cu") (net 3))
 (segment (start 40.7964 18.9008) (end 42.8665 20.9709) (width 0.2) (layer "F.Cu") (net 3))
 (segment (start 30 11.2) (end 32 11.2) (width 0.2) (layer "F.Cu") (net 3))
 (segment (start 28.1926 34.8028) (end 32.6616 30.3338) (width 0.2) (layer "F.Cu") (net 3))
 (segment (start 38.1936 15.2) (end 40.7964 17.8028) (width 0.2) (layer "F.Cu") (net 3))
 (segment (start 40.6972 19) (end 35.0569 19) (width 0.2) (layer "F.Cu") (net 3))
 (segment (start 36.4504 24.2) (end 36.4504 23.9237) (width 0.2) (layer "F.Cu") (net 3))
 (segment (start 36 15.2) (end 38.1936 15.2) (width 0.2) (layer "F.Cu") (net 3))
 (segment (start 23.0028 34.8028) (end 28.1926 34.8028) (width 0.2) (layer "F.Cu") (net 3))
 (segment (start 32.6616 30.3338) (end 32.6616 27.9888) (width 0.2) (layer "F.Cu") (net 3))
 (segment (start 35.0569 19) (end 33.5502 20.5067) (width 0.2) (layer "F.Cu") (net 3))
 (segment (start 32.75 21.025) (end 33.5502 21.025) (width 0.2) (layer "F.Cu") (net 3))
 (segment (start 12.58 22.78) (end 12.08 22.78) (width 0.2) (layer "F.Cu") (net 4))
 (segment (start 26.2 34) (end 24.2 32) (width 0.2) (layer "F.Cu") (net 4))
 (segment (start 24.2 32) (end 21.8 32) (width 0.2) (layer "F.Cu") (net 4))
 (segment (start 21.8 32) (end 12.58 22.78) (width 0.2) (layer "F.Cu") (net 4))
 (segment (start 27 33.2) (end 27.8 34) (width 0.2) (layer "F.Cu") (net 9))
 (segment (start 24.2 24) (end 24.4623 24) (width 0.2) (layer "F.Cu") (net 9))
 (segment (start 24.5322 24.0699) (end 26.2771 22.325) (width 0.2) (layer "F.Cu") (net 9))
 (segment (start 26.2771 22.325) (end 28.4483 22.325) (width 0.2) (layer "F.Cu") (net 9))
 (segment (start 24.4623 24) (end 24.5322 24.0699) (width 0.2) (layer "F.Cu") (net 9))
 (segment (start 27 26.5377) (end 27 33.2) (width 0.2) (layer "F.Cu") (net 9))
 (segment (start 29.25 22.325) (end 28.4483 22.325) (width 0.2) (layer "F.Cu") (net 9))
 (segment (start 24.5322 24.0699) (end 27 26.5377) (width 0.2) (layer "F.Cu") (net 9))
 (segment (start 34.3911 18.2) (end 31.9483 20.6428) (width 0.2) (layer "F.Cu") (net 6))
 (segment (start 36 16.8) (end 36 18.2) (width 0.2) (layer "F.Cu") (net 6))
 (segment (start 27.8 27) (end 27.8 26) (width 0.2) (layer "F.Cu") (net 6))
 (segment (start 31.9483 20.6428) (end 31.9483 22.975) (width 0.2) (layer "F.Cu") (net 6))
 (segment (start 40 18.2) (end 36 18.2) (width 0.2) (layer "F.Cu") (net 6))
 (segment (start 32.75 22.975) (end 31.9483 22.975) (width 0.2) (layer "F.Cu") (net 6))
 (segment (start 28.9233 26) (end 31.9483 22.975) (width 0.2) (layer "F.Cu") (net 6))
 (segment (start 27.8 26) (end 28.9233 26) (width 0.2) (layer "F.Cu") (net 6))
 (segment (start 36 18.2) (end 34.3911 18.2) (width 0.2) (layer "F.Cu") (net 6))
 (segment (start 27.8 26) (end 25.8 24) (width 0.2) (layer "F.Cu") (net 6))
 (segment (start 27.8 21.0267) (end 28.4483 21.675) (width 0.2) (layer "F.Cu") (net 12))
 (segment (start 27.8 19) (end 27.8 21.0267) (width 0.2) (layer "F.Cu") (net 12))
 (segment (start 25.9771 21.0267) (end 27.8 21.0267) (width 0.2) (layer "F.Cu") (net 12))
 (segment (start 23.4708 24.4599) (end 23.4708 23.533) (width 0.2) (layer "F.Cu") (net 12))
 (segment (start 26.0109 27) (end 23.4708 24.4599) (width 0.2) (layer "F.Cu") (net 12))
 (segment (start 23.4708 23.533) (end 25.9771 21.0267) (width 0.2) (layer "F.Cu") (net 12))
 (segment (start 26.2 27) (end 26.0109 27) (width 0.2) (layer "F.Cu") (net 12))
 (segment (start 29.25 21.675) (end 28.4483 21.675) (width 0.2) (layer "F.Cu") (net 12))
 (segment (start 30.7775 15.6897) (end 30.7775 12.3725) (width 0.2) (layer "F.Cu") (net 11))
 (segment (start 29.5857 11.997) (end 29.2032 11.6145) (width 0.2) (layer "F.Cu") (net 11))
 (segment (start 29.25 21.025) (end 28.4483 21.025) (width 0.2) (layer "F.Cu") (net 11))
 (segment (start 29.5175 10.4621) (end 36.6621 10.4621) (width 0.2) (layer "F.Cu") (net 11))
 (segment (start 26.2 19) (end 26.989 18.211) (width 0.2) (layer "F.Cu") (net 11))
 (segment (start 26.989 18.211) (end 28.2562 18.211) (width 0.2) (layer "F.Cu") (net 11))
 (segment (start 29.2032 10.7764) (end 29.5175 10.4621) (width 0.2) (layer "F.Cu") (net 11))
 (segment (start 30.402 11.997) (end 29.5857 11.997) (width 0.2) (layer "F.Cu") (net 11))
 (segment (start 28.4483 20.5233) (end 28.4483 21.025) (width 0.2) (layer "F.Cu") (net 11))
 (segment (start 29.2032 11.6145) (end 29.2032 10.7764) (width 0.2) (layer "F.Cu") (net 11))
 (segment (start 28.5486 20.423) (end 28.4483 20.5233) (width 0.2) (layer "F.Cu") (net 11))
 (segment (start 28.2562 18.211) (end 28.5486 18.5034) (width 0.2) (layer "F.Cu") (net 11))
 (segment (start 28.5486 18.5034) (end 28.5486 20.423) (width 0.2) (layer "F.Cu") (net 11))
 (segment (start 36.6621 10.4621) (end 37.2 11) (width 0.2) (layer "F.Cu") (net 11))
 (segment (start 30.7775 12.3725) (end 30.402 11.997) (width 0.2) (layer "F.Cu") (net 11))
 (segment (start 28.2562 18.211) (end 30.7775 15.6897) (width 0.2) (layer "F.Cu") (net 11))
 (segment (start 42 9.215) (end 46.835 4.38) (width 0.2) (layer "F.Cu") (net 10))
 (segment (start 42.8263 12.1947) (end 42.4625 12.5585) (width 0.2) (layer "F.Cu") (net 10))
 (segment (start 40.3585 12.5585) (end 38.8 11) (width 0.2) (layer "F.Cu") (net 10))
 (segment (start 42 10.2) (end 42.8263 11.0263) (width 0.2) (layer "F.Cu") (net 10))
 (segment (start 42 10.2) (end 42 9.215) (width 0.2) (layer "F.Cu") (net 10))
 (segment (start 42.4625 12.5585) (end 40.3585 12.5585) (width 0.2) (layer "F.Cu") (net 10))
 (segment (start 42.8263 11.0263) (end 42.8263 12.1947) (width 0.2) (layer "F.Cu") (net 10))
 (segment (start 6.5642 23.8925) (end 8.9355 23.8925) (width 0.2) (layer "F.Cu") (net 8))
 (segment (start 21.2 10) (end 9.5917 10) (width 0.2) (layer "F.Cu") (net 8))
 (segment (start 2.0333 17.5584) (end 2.0333 19.3616) (width 0.2) (layer "F.Cu") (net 8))
 (segment (start 8.9355 23.8925) (end 10.048 22.78) (width 0.2) (layer "F.Cu") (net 8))
 (segment (start 9.5917 10) (end 2.0333 17.5584) (width 0.2) (layer "F.Cu") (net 8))
 (segment (start 2.0333 19.3616) (end 6.5642 23.8925) (width 0.2) (layer "F.Cu") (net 8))
 (segment (start 38 10.5232) (end 38 11.452) (width 0.2) (layer "F.Cu") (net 5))
 (segment (start 28.8015 12.2) (end 28.8015 10.5978) (width 0.2) (layer "F.Cu") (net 5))
 (segment (start 29.3424 10.0569) (end 37.5337 10.0569) (width 0.2) (layer "F.Cu") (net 5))
 (segment (start 28.8015 10.5978) (end 29.3424 10.0569) (width 0.2) (layer "F.Cu") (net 5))
 (segment (start 46.168 19.62) (end 46.835 19.62) (width 0.2) (layer "F.Cu") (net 5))
 (segment (start 29.4015 12.8) (end 28.8015 12.2) (width 0.2) (layer "F.Cu") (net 5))
 (segment (start 25 12.2) (end 28.8015 12.2) (width 0.2) (layer "F.Cu") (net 5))
 (segment (start 38 11.452) (end 46.168 19.62) (width 0.2) (layer "F.Cu") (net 5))
 (segment (start 25 12.2) (end 22.8 10) (width 0.2) (layer "F.Cu") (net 5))
 (segment (start 30 12.8) (end 29.4015 12.8) (width 0.2) (layer "F.Cu") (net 5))
 (segment (start 37.5337 10.0569) (end 38 10.5232) (width 0.2) (layer "F.Cu") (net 5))
 (segment (start 55.2 19.8) (end 63 12) (width 0.2) (layer "F.Cu") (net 1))
 (segment (start 55.2 28) (end 55.2 19.8) (width 0.2) (layer "F.Cu") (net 1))
 (segment (start 59.2 28) (end 56.8 28) (width 0.2) (layer "F.Cu") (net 2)))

